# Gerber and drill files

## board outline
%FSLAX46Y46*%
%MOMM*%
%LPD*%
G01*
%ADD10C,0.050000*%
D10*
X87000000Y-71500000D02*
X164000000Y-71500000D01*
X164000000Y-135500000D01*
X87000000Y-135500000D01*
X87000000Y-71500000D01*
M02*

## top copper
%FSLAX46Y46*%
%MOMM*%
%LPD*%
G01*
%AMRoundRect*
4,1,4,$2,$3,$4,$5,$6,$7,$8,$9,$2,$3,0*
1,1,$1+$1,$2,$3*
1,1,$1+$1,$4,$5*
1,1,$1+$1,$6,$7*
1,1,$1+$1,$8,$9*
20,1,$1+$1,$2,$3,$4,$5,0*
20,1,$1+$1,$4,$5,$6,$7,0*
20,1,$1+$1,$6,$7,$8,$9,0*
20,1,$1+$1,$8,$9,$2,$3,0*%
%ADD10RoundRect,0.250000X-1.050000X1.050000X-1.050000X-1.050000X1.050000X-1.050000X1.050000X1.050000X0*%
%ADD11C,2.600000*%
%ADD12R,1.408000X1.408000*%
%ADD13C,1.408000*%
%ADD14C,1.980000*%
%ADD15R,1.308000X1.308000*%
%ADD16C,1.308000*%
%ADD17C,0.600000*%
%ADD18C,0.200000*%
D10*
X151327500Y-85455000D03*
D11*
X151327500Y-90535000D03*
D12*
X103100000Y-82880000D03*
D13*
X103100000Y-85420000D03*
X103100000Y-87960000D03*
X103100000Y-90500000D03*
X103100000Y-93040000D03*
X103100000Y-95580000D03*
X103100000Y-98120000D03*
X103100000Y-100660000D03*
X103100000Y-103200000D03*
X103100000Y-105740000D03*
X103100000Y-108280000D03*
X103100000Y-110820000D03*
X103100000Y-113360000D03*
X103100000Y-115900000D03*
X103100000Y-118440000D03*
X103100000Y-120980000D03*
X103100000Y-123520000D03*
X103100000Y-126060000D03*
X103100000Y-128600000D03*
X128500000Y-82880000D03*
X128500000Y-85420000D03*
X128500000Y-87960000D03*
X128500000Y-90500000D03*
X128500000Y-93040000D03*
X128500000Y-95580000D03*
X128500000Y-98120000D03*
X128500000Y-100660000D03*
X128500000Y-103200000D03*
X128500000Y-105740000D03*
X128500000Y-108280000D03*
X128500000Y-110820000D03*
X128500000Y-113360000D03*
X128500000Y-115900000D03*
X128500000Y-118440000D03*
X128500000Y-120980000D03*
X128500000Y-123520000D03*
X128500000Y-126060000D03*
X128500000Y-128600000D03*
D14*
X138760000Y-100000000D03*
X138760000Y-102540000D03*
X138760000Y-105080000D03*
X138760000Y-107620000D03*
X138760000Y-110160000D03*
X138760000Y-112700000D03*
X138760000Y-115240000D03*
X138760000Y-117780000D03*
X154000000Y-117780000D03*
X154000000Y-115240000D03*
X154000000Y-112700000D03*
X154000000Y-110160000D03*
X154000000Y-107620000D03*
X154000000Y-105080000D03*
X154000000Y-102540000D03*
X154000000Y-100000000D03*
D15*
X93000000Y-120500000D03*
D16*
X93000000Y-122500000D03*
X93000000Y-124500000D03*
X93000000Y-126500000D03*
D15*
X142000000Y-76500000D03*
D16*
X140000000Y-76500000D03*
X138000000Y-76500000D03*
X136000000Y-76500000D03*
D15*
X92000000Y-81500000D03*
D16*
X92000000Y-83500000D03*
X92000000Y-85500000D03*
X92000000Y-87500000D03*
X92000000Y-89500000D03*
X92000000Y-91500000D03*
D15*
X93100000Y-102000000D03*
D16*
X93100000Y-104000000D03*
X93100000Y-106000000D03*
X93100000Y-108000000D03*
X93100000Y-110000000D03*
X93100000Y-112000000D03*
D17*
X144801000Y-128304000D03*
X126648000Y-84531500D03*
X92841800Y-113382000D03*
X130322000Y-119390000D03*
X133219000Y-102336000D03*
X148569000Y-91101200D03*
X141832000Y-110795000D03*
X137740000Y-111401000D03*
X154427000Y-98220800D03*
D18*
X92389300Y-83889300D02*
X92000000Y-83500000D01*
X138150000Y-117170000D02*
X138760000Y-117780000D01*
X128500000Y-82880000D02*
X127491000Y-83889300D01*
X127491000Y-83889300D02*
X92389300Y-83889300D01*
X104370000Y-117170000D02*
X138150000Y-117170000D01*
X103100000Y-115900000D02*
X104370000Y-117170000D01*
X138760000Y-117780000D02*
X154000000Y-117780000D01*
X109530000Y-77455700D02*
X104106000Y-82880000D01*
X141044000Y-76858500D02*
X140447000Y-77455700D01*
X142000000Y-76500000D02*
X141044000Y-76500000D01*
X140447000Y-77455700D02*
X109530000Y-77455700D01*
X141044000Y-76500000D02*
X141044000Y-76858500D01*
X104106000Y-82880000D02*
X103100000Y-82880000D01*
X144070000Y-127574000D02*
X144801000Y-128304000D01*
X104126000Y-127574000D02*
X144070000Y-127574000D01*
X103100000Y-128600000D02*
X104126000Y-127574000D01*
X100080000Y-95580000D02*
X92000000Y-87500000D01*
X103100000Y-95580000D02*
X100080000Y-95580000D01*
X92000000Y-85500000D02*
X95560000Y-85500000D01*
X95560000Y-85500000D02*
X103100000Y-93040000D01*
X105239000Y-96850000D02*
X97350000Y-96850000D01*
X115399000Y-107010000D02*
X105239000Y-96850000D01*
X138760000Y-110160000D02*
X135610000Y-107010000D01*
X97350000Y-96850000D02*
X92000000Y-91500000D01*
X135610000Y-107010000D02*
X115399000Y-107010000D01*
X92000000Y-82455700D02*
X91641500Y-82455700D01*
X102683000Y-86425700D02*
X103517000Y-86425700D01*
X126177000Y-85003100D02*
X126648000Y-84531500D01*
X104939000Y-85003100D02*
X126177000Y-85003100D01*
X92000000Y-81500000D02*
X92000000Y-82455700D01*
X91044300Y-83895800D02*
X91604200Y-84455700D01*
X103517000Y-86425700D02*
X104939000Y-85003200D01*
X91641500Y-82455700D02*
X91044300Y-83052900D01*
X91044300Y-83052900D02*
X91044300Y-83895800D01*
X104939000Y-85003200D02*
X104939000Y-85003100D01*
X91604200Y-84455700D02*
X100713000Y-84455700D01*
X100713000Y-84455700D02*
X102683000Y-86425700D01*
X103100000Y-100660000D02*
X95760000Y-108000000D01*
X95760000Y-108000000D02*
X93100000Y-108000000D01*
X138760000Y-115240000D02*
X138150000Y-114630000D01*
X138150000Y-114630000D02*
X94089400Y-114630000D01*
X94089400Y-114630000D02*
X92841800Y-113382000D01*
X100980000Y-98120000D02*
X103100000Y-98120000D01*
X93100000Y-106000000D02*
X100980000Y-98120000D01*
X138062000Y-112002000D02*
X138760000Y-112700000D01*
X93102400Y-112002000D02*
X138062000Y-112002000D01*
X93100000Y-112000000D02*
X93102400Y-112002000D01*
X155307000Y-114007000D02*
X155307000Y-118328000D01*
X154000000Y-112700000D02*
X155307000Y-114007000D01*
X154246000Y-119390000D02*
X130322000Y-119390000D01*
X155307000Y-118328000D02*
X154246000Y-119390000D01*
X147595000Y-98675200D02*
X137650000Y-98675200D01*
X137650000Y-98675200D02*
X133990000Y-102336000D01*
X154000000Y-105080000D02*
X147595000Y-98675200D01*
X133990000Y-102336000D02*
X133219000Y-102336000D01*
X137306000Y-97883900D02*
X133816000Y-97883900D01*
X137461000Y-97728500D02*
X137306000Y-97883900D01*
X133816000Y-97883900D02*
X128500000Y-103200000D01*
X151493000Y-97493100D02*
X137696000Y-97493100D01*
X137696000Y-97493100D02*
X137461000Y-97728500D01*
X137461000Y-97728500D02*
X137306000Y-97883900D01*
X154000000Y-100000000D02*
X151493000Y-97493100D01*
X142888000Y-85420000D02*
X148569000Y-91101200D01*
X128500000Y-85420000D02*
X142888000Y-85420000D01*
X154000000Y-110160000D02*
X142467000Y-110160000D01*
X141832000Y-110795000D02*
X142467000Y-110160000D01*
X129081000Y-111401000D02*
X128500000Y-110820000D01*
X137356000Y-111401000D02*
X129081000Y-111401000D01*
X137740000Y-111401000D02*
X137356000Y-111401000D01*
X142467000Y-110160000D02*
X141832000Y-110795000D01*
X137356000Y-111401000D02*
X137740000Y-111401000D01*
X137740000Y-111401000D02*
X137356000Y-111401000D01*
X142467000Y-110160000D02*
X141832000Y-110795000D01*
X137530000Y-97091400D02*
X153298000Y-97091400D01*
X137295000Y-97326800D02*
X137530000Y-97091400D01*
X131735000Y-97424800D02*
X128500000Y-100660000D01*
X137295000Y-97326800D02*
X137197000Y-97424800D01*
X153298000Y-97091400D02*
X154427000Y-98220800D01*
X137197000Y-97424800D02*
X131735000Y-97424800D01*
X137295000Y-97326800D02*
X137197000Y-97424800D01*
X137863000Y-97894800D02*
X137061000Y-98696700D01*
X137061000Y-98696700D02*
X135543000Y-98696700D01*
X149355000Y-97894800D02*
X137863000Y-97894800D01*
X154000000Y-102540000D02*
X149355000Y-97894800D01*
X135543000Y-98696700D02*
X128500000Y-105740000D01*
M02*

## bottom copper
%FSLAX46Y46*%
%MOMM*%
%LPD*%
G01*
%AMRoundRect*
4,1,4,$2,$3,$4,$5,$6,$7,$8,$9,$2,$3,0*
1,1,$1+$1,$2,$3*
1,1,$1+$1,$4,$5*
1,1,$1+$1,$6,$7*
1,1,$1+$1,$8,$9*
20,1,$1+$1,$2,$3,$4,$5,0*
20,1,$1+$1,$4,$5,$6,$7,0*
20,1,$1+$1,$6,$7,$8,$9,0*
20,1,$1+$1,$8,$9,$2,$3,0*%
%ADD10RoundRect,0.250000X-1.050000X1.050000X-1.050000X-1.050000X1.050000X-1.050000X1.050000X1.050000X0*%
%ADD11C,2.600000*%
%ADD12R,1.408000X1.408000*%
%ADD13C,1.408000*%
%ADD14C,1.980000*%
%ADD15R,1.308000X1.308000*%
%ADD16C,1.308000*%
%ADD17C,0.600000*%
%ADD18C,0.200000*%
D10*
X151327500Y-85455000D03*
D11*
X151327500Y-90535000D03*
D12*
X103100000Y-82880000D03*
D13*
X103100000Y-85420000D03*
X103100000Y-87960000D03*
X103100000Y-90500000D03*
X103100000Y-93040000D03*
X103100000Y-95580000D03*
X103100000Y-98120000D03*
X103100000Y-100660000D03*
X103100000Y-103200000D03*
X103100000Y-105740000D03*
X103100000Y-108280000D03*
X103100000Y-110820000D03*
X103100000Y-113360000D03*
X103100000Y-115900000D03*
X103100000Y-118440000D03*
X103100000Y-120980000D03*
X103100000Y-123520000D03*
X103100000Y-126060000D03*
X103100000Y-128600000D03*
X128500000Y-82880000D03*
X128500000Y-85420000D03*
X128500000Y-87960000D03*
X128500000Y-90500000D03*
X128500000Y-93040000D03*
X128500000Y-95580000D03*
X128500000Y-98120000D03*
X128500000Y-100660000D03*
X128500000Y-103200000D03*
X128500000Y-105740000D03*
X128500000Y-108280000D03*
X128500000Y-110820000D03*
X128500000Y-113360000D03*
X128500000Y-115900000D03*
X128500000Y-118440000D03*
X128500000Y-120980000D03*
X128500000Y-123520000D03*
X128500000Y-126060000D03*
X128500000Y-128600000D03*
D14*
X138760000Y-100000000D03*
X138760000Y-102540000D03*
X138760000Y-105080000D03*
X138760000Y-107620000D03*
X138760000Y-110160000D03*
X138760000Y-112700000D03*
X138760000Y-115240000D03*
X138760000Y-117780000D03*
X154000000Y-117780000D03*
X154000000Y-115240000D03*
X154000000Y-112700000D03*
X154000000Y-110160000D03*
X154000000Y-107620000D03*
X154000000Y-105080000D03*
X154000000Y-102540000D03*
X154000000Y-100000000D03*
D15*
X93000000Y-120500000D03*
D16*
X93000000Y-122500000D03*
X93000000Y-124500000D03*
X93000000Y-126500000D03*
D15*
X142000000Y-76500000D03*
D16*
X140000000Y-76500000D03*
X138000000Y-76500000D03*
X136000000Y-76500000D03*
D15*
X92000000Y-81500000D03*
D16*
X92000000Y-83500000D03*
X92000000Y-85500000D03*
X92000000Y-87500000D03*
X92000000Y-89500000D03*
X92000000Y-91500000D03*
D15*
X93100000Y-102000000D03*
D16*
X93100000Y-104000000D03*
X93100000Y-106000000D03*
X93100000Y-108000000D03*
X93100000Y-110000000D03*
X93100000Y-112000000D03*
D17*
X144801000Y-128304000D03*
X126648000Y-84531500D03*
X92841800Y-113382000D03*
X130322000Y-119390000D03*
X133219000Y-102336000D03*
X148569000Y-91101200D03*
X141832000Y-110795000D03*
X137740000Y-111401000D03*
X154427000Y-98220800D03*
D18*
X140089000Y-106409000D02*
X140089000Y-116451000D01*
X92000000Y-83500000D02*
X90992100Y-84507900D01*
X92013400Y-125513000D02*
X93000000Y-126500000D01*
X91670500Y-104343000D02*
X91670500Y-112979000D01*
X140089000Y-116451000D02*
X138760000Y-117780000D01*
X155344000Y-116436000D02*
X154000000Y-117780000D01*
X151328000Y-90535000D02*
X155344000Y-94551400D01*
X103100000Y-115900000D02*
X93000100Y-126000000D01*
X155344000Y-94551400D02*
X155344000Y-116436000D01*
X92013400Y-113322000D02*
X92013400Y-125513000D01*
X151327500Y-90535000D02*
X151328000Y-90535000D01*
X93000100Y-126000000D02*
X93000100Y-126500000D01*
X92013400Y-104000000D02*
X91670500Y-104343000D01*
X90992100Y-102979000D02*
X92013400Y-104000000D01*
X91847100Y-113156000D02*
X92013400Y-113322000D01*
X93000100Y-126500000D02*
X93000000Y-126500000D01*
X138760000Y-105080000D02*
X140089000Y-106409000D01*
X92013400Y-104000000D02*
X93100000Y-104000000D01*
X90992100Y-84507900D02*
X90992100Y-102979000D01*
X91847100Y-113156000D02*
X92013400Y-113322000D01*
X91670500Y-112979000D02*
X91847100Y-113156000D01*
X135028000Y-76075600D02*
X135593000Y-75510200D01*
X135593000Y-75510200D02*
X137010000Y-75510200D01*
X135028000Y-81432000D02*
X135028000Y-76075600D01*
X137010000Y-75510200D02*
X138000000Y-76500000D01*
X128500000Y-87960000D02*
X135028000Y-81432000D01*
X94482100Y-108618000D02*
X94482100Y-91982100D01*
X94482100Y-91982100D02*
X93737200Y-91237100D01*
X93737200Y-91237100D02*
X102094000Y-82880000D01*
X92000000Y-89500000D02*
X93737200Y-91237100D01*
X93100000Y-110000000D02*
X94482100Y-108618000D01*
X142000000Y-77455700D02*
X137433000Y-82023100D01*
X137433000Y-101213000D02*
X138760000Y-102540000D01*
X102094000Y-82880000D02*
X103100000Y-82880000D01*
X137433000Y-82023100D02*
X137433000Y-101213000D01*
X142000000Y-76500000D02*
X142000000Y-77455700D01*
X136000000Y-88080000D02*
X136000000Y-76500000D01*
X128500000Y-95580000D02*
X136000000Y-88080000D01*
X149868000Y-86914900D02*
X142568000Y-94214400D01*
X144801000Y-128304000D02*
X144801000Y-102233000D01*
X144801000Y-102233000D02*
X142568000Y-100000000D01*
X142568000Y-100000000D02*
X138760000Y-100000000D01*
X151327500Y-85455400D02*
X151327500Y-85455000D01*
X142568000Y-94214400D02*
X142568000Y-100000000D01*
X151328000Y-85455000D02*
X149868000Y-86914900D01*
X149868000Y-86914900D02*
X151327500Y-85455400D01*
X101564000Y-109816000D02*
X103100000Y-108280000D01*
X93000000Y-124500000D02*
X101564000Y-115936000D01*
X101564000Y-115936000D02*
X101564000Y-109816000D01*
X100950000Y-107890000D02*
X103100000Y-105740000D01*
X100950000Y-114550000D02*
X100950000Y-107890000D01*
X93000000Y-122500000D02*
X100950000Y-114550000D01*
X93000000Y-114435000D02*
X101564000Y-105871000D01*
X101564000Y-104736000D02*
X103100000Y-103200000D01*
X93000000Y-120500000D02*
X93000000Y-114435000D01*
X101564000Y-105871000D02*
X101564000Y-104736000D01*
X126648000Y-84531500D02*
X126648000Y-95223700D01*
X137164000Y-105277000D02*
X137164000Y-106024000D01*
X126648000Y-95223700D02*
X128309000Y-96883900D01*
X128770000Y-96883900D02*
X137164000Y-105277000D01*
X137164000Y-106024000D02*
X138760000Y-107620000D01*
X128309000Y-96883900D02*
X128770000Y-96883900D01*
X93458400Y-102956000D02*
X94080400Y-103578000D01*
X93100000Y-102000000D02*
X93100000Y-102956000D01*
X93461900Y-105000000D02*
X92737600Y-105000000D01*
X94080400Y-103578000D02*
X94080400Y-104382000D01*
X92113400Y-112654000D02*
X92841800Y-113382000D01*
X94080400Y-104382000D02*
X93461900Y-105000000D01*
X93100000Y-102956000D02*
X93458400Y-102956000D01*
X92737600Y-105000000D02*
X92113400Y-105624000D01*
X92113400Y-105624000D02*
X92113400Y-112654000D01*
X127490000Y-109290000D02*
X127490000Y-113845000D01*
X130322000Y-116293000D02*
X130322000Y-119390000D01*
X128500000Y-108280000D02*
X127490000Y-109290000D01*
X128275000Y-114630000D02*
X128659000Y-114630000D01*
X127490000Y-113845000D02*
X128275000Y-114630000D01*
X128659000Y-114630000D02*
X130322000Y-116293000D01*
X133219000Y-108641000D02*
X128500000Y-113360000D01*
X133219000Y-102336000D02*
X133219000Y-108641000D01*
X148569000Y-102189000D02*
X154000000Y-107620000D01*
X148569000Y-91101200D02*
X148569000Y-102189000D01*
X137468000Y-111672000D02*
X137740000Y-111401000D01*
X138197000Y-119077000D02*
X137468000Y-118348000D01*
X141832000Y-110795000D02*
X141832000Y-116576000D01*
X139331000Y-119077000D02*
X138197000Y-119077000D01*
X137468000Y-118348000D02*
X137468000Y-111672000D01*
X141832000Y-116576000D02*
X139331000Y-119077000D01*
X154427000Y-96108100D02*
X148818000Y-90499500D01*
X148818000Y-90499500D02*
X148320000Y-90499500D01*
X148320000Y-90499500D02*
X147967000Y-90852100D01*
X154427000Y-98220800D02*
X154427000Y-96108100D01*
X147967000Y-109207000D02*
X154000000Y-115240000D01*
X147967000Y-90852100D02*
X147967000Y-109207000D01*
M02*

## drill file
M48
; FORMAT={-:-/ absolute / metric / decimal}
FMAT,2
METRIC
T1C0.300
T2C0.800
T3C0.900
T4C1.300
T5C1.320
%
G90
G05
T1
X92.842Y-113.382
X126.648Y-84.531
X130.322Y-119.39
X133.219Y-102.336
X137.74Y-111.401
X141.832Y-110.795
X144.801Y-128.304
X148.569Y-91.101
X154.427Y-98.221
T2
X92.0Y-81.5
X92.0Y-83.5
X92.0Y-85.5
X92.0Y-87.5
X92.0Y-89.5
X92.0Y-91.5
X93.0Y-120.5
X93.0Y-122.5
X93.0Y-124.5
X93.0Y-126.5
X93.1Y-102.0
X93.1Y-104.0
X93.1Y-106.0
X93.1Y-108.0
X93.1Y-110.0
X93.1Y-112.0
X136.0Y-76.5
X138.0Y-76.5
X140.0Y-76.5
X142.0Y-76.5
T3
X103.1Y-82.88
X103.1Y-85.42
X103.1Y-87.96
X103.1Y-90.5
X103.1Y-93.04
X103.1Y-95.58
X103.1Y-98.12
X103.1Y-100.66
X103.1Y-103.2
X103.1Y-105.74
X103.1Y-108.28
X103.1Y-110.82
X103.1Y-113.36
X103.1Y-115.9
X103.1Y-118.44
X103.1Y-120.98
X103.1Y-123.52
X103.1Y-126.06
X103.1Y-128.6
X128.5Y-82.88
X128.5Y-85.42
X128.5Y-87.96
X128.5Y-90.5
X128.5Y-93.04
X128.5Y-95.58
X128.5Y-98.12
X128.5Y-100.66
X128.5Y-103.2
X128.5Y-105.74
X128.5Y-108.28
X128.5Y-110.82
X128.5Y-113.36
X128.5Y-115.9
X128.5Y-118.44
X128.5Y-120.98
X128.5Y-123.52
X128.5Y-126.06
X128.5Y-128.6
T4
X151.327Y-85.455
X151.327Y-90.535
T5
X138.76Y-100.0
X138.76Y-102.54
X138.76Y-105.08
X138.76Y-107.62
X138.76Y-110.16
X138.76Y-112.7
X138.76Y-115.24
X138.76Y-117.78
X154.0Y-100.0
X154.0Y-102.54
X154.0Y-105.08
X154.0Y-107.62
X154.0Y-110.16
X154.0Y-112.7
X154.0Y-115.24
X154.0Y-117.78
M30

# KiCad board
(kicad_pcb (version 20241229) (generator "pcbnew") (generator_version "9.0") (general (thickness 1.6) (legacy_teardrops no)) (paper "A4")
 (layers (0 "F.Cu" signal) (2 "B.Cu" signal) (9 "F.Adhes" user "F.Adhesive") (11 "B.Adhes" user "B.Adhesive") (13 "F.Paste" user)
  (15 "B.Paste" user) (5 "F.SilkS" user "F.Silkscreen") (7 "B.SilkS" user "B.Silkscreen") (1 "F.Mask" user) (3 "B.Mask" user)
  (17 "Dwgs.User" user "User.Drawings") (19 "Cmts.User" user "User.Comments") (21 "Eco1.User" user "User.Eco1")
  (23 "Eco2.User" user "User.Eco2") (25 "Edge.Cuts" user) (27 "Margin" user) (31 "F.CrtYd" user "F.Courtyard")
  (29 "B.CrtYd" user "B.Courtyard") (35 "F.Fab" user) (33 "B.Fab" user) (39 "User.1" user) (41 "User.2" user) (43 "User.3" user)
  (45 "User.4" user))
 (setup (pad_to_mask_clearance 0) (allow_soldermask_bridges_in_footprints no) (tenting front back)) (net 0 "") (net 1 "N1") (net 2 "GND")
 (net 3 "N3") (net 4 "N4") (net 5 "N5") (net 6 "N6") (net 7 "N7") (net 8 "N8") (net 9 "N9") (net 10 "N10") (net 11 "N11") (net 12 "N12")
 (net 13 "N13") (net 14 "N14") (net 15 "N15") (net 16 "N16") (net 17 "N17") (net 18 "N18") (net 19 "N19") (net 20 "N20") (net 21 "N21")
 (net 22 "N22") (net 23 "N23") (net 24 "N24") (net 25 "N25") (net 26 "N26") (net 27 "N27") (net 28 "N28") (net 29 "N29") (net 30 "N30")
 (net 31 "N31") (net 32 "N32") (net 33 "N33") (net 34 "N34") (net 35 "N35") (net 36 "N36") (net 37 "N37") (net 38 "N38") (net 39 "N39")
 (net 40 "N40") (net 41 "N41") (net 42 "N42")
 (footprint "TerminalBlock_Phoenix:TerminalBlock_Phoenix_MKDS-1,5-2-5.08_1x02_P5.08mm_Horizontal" (layer "F.Cu") (at 151.3275 85.455 -90)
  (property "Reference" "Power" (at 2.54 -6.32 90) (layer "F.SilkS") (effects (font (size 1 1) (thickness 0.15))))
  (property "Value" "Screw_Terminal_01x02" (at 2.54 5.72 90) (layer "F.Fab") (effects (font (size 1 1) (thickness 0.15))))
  (pad "1" thru_hole roundrect (at 0 0 270) (size 2.6 2.6) (drill 1.3) (layers "*.Cu" "*.Mask") (remove_unused_layers no)
   (roundrect_rratio 0.096154) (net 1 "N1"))
  (pad "2" thru_hole circle (at 5.08 0 270) (size 2.6 2.6) (drill 1.3) (layers "*.Cu" "*.Mask") (remove_unused_layers no) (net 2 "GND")))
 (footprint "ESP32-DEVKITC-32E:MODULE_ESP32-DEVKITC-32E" (layer "F.Cu") (at 115.8 105.715)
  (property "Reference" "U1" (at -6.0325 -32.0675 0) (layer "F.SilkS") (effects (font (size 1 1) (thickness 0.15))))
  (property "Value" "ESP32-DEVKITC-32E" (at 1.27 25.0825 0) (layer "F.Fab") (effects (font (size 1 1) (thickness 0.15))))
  (pad "J2_1" thru_hole rect (at -12.7 -22.835) (size 1.408 1.408) (drill 0.9) (layers "*.Cu" "*.Mask") (remove_unused_layers no)
   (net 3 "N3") (solder_mask_margin 0.102))
  (pad "J2_2" thru_hole circle (at -12.7 -20.295) (size 1.408 1.408) (drill 0.9) (layers "*.Cu" "*.Mask") (remove_unused_layers no)
   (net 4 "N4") (solder_mask_margin 0.102))
  (pad "J2_3" thru_hole circle (at -12.7 -17.755) (size 1.408 1.408) (drill 0.9) (layers "*.Cu" "*.Mask") (remove_unused_layers no)
   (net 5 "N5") (solder_mask_margin 0.102))
  (pad "J2_4" thru_hole circle (at -12.7 -15.215) (size 1.408 1.408) (drill 0.9) (layers "*.Cu" "*.Mask") (remove_unused_layers no)
   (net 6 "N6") (solder_mask_margin 0.102))
  (pad "J2_5" thru_hole circle (at -12.7 -12.675) (size 1.408 1.408) (drill 0.9) (layers "*.Cu" "*.Mask") (remove_unused_layers no)
   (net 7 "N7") (solder_mask_margin 0.102))
  (pad "J2_6" thru_hole circle (at -12.7 -10.135) (size 1.408 1.408) (drill 0.9) (layers "*.Cu" "*.Mask") (remove_unused_layers no)
   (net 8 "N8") (solder_mask_margin 0.102))
  (pad "J2_7" thru_hole circle (at -12.7 -7.595) (size 1.408 1.408) (drill 0.9) (layers "*.Cu" "*.Mask") (remove_unused_layers no)
   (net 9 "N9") (solder_mask_margin 0.102))
  (pad "J2_8" thru_hole circle (at -12.7 -5.055) (size 1.408 1.408) (drill 0.9) (layers "*.Cu" "*.Mask") (remove_unused_layers no)
   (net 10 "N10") (solder_mask_margin 0.102))
  (pad "J2_9" thru_hole circle (at -12.7 -2.515) (size 1.408 1.408) (drill 0.9) (layers "*.Cu" "*.Mask") (remove_unused_layers no)
   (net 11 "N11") (solder_mask_margin 0.102))
  (pad "J2_10" thru_hole circle (at -12.7 0.025) (size 1.408 1.408) (drill 0.9) (layers "*.Cu" "*.Mask") (remove_unused_layers no)
   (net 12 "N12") (solder_mask_margin 0.102))
  (pad "J2_11" thru_hole circle (at -12.7 2.565) (size 1.408 1.408) (drill 0.9) (layers "*.Cu" "*.Mask") (remove_unused_layers no)
   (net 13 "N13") (solder_mask_margin 0.102))
  (pad "J2_12" thru_hole circle (at -12.7 5.105) (size 1.408 1.408) (drill 0.9) (layers "*.Cu" "*.Mask") (remove_unused_layers no)
   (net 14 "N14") (solder_mask_margin 0.102))
  (pad "J2_13" thru_hole circle (at -12.7 7.645) (size 1.408 1.408) (drill 0.9) (layers "*.Cu" "*.Mask") (remove_unused_layers no)
   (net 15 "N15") (solder_mask_margin 0.102))
  (pad "J2_14" thru_hole circle (at -12.7 10.185) (size 1.408 1.408) (drill 0.9) (layers "*.Cu" "*.Mask") (remove_unused_layers no)
   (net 2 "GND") (solder_mask_margin 0.102))
  (pad "J2_15" thru_hole circle (at -12.7 12.725) (size 1.408 1.408) (drill 0.9) (layers "*.Cu" "*.Mask") (remove_unused_layers no)
   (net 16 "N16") (solder_mask_margin 0.102))
  (pad "J2_16" thru_hole circle (at -12.7 15.265) (size 1.408 1.408) (drill 0.9) (layers "*.Cu" "*.Mask") (remove_unused_layers no)
   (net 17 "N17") (solder_mask_margin 0.102))
  (pad "J2_17" thru_hole circle (at -12.7 17.805) (size 1.408 1.408) (drill 0.9) (layers "*.Cu" "*.Mask") (remove_unused_layers no)
   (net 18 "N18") (solder_mask_margin 0.102))
  (pad "J2_18" thru_hole circle (at -12.7 20.345) (size 1.408 1.408) (drill 0.9) (layers "*.Cu" "*.Mask") (remove_unused_layers no)
   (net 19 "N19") (solder_mask_margin 0.102))
  (pad "J2_19" thru_hole circle (at -12.7 22.885) (size 1.408 1.408) (drill 0.9) (layers "*.Cu" "*.Mask") (remove_unused_layers no)
   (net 1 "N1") (solder_mask_margin 0.102))
  (pad "J3_1" thru_hole circle (at 12.7 -22.835) (size 1.408 1.408) (drill 0.9) (layers "*.Cu" "*.Mask") (remove_unused_layers no)
   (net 2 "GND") (solder_mask_margin 0.102))
  (pad "J3_2" thru_hole circle (at 12.7 -20.295) (size 1.408 1.408) (drill 0.9) (layers "*.Cu" "*.Mask") (remove_unused_layers no)
   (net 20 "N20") (solder_mask_margin 0.102))
  (pad "J3_3" thru_hole circle (at 12.7 -17.755) (size 1.408 1.408) (drill 0.9) (layers "*.Cu" "*.Mask") (remove_unused_layers no)
   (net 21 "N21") (solder_mask_margin 0.102))
  (pad "J3_4" thru_hole circle (at 12.7 -15.215) (size 1.408 1.408) (drill 0.9) (layers "*.Cu" "*.Mask") (remove_unused_layers no)
   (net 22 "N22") (solder_mask_margin 0.102))
  (pad "J3_5" thru_hole circle (at 12.7 -12.675) (size 1.408 1.408) (drill 0.9) (layers "*.Cu" "*.Mask") (remove_unused_layers no)
   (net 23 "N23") (solder_mask_margin 0.102))
  (pad "J3_6" thru_hole circle (at 12.7 -10.135) (size 1.408 1.408) (drill 0.9) (layers "*.Cu" "*.Mask") (remove_unused_layers no)
   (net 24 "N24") (solder_mask_margin 0.102))
  (pad "J3_7" thru_hole circle (at 12.7 -7.595) (size 1.408 1.408) (drill 0.9) (layers "*.Cu" "*.Mask") (remove_unused_layers no)
   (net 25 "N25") (solder_mask_margin 0.102))
  (pad "J3_8" thru_hole circle (at 12.7 -5.055) (size 1.408 1.408) (drill 0.9) (layers "*.Cu" "*.Mask") (remove_unused_layers no)
   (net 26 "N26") (solder_mask_margin 0.102))
  (pad "J3_9" thru_hole circle (at 12.7 -2.515) (size 1.408 1.408) (drill 0.9) (layers "*.Cu" "*.Mask") (remove_unused_layers no)
   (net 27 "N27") (solder_mask_margin 0.102))
  (pad "J3_10" thru_hole circle (at 12.7 0.025) (size 1.408 1.408) (drill 0.9) (layers "*.Cu" "*.Mask") (remove_unused_layers no)
   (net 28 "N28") (solder_mask_margin 0.102))
  (pad "J3_11" thru_hole circle (at 12.7 2.565) (size 1.408 1.408) (drill 0.9) (layers "*.Cu" "*.Mask") (remove_unused_layers no)
   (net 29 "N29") (solder_mask_margin 0.102))
  (pad "J3_12" thru_hole circle (at 12.7 5.105) (size 1.408 1.408) (drill 0.9) (layers "*.Cu" "*.Mask") (remove_unused_layers no)
   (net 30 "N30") (solder_mask_margin 0.102))
  (pad "J3_13" thru_hole circle (at 12.7 7.645) (size 1.408 1.408) (drill 0.9) (layers "*.Cu" "*.Mask") (remove_unused_layers no)
   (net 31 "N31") (solder_mask_margin 0.102))
  (pad "J3_14" thru_hole circle (at 12.7 10.185) (size 1.408 1.408) (drill 0.9) (layers "*.Cu" "*.Mask") (remove_unused_layers no)
   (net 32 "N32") (solder_mask_margin 0.102))
  (pad "J3_15" thru_hole circle (at 12.7 12.725) (size 1.408 1.408) (drill 0.9) (layers "*.Cu" "*.Mask") (remove_unused_layers no)
   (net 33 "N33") (solder_mask_margin 0.102))
  (pad "J3_16" thru_hole circle (at 12.7 15.265) (size 1.408 1.408) (drill 0.9) (layers "*.Cu" "*.Mask") (remove_unused_layers no)
   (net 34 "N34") (solder_mask_margin 0.102))
  (pad "J3_17" thru_hole circle (at 12.7 17.805) (size 1.408 1.408) (drill 0.9) (layers "*.Cu" "*.Mask") (remove_unused_layers no)
   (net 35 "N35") (solder_mask_margin 0.102))
  (pad "J3_18" thru_hole circle (at 12.7 20.345) (size 1.408 1.408) (drill 0.9) (layers "*.Cu" "*.Mask") (remove_unused_layers no)
   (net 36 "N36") (solder_mask_margin 0.102))
  (pad "J3_19" thru_hole circle (at 12.7 22.885) (size 1.408 1.408) (drill 0.9) (layers "*.Cu" "*.Mask") (remove_unused_layers no)
   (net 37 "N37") (solder_mask_margin 0.102)))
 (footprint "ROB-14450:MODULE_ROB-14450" (layer "F.Cu") (at 146.38 108.89)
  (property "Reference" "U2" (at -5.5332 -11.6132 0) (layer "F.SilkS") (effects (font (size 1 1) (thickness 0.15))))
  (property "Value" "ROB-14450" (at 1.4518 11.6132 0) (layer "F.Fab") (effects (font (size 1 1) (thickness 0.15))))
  (pad "1" thru_hole circle (at -7.62 -8.89) (size 1.98 1.98) (drill 1.32) (layers "*.Cu" "*.Mask") (remove_unused_layers no) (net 1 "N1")
   (solder_mask_margin 0.102))
  (pad "2" thru_hole circle (at -7.62 -6.35) (size 1.98 1.98) (drill 1.32) (layers "*.Cu" "*.Mask") (remove_unused_layers no) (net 3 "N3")
   (solder_mask_margin 0.102))
  (pad "3" thru_hole circle (at -7.62 -3.81) (size 1.98 1.98) (drill 1.32) (layers "*.Cu" "*.Mask") (remove_unused_layers no) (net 2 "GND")
   (solder_mask_margin 0.102))
  (pad "4" thru_hole circle (at -7.62 -1.27) (size 1.98 1.98) (drill 1.32) (layers "*.Cu" "*.Mask") (remove_unused_layers no) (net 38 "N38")
   (solder_mask_margin 0.102))
  (pad "5" thru_hole circle (at -7.62 1.27) (size 1.98 1.98) (drill 1.32) (layers "*.Cu" "*.Mask") (remove_unused_layers no) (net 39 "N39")
   (solder_mask_margin 0.102))
  (pad "6" thru_hole circle (at -7.62 3.81) (size 1.98 1.98) (drill 1.32) (layers "*.Cu" "*.Mask") (remove_unused_layers no) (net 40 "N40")
   (solder_mask_margin 0.102))
  (pad "7" thru_hole circle (at -7.62 6.35) (size 1.98 1.98) (drill 1.32) (layers "*.Cu" "*.Mask") (remove_unused_layers no) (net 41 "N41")
   (solder_mask_margin 0.102))
  (pad "8" thru_hole circle (at -7.62 8.89) (size 1.98 1.98) (drill 1.32) (layers "*.Cu" "*.Mask") (remove_unused_layers no) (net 2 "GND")
   (solder_mask_margin 0.102))
  (pad "9" thru_hole circle (at 7.62 8.89) (size 1.98 1.98) (drill 1.32) (layers "*.Cu" "*.Mask") (remove_unused_layers no) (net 2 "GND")
   (solder_mask_margin 0.102))
  (pad "10" thru_hole circle (at 7.62 6.35) (size 1.98 1.98) (drill 1.32) (layers "*.Cu" "*.Mask") (remove_unused_layers no) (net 26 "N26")
   (solder_mask_margin 0.102))
  (pad "11" thru_hole circle (at 7.62 3.81) (size 1.98 1.98) (drill 1.32) (layers "*.Cu" "*.Mask") (remove_unused_layers no) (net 29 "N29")
   (solder_mask_margin 0.102))
  (pad "12" thru_hole circle (at 7.62 1.27) (size 1.98 1.98) (drill 1.32) (layers "*.Cu" "*.Mask") (remove_unused_layers no) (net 30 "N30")
   (solder_mask_margin 0.102))
  (pad "13" thru_hole circle (at 7.62 -1.27) (size 1.98 1.98) (drill 1.32) (layers "*.Cu" "*.Mask") (remove_unused_layers no) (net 20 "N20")
   (solder_mask_margin 0.102))
  (pad "14" thru_hole circle (at 7.62 -3.81) (size 1.98 1.98) (drill 1.32) (layers "*.Cu" "*.Mask") (remove_unused_layers no) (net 31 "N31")
   (solder_mask_margin 0.102))
  (pad "15" thru_hole circle (at 7.62 -6.35) (size 1.98 1.98) (drill 1.32) (layers "*.Cu" "*.Mask") (remove_unused_layers no) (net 28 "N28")
   (solder_mask_margin 0.102))
  (pad "16" thru_hole circle (at 7.62 -8.89) (size 1.98 1.98) (drill 1.32) (layers "*.Cu" "*.Mask") (remove_unused_layers no) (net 27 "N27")
   (solder_mask_margin 0.102)))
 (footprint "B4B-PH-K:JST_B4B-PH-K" (layer "F.Cu") (at 92.45 123.5 90)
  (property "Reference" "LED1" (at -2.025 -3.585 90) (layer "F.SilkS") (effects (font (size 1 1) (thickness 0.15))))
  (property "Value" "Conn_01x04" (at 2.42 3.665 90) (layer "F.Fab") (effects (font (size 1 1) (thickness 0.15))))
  (pad "1" thru_hole rect (at 3 0.55 90) (size 1.308 1.308) (drill 0.8) (layers "*.Cu" "*.Mask") (remove_unused_layers no) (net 11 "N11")
   (solder_mask_margin 0.102))
  (pad "2" thru_hole circle (at 1 0.55 90) (size 1.308 1.308) (drill 0.8) (layers "*.Cu" "*.Mask") (remove_unused_layers no) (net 12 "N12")
   (solder_mask_margin 0.102))
  (pad "3" thru_hole circle (at -1 0.55 90) (size 1.308 1.308) (drill 0.8) (layers "*.Cu" "*.Mask") (remove_unused_layers no) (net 13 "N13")
   (solder_mask_margin 0.102))
  (pad "4" thru_hole circle (at -3 0.55 90) (size 1.308 1.308) (drill 0.8) (layers "*.Cu" "*.Mask") (remove_unused_layers no) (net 2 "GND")
   (solder_mask_margin 0.102)))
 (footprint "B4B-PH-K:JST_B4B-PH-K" (layer "F.Cu") (at 139 75.95)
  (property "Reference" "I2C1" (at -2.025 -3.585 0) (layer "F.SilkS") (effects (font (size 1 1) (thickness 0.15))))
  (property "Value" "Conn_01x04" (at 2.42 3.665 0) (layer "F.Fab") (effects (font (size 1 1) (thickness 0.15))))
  (pad "1" thru_hole rect (at 3 0.55) (size 1.308 1.308) (drill 0.8) (layers "*.Cu" "*.Mask") (remove_unused_layers no) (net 3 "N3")
   (solder_mask_margin 0.102))
  (pad "2" thru_hole circle (at 1 0.55) (size 1.308 1.308) (drill 0.8) (layers "*.Cu" "*.Mask") (remove_unused_layers no) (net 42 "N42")
   (solder_mask_margin 0.102))
  (pad "3" thru_hole circle (at -1 0.55) (size 1.308 1.308) (drill 0.8) (layers "*.Cu" "*.Mask") (remove_unused_layers no) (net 21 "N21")
   (solder_mask_margin 0.102))
  (pad "4" thru_hole circle (at -3 0.55) (size 1.308 1.308) (drill 0.8) (layers "*.Cu" "*.Mask") (remove_unused_layers no) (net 24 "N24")
   (solder_mask_margin 0.102)))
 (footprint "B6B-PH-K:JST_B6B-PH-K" (layer "F.Cu") (at 91.45 86.5 90)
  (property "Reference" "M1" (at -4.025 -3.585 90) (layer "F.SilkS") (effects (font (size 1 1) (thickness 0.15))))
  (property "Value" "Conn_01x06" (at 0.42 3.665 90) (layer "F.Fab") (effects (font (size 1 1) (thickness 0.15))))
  (pad "1" thru_hole rect (at 5 0.55 90) (size 1.308 1.308) (drill 0.8) (layers "*.Cu" "*.Mask") (remove_unused_layers no) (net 38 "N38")
   (solder_mask_margin 0.102))
  (pad "2" thru_hole circle (at 3 0.55 90) (size 1.308 1.308) (drill 0.8) (layers "*.Cu" "*.Mask") (remove_unused_layers no) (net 2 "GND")
   (solder_mask_margin 0.102))
  (pad "3" thru_hole circle (at 1 0.55 90) (size 1.308 1.308) (drill 0.8) (layers "*.Cu" "*.Mask") (remove_unused_layers no) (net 7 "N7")
   (solder_mask_margin 0.102))
  (pad "4" thru_hole circle (at -1 0.55 90) (size 1.308 1.308) (drill 0.8) (layers "*.Cu" "*.Mask") (remove_unused_layers no) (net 8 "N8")
   (solder_mask_margin 0.102))
  (pad "5" thru_hole circle (at -3 0.55 90) (size 1.308 1.308) (drill 0.8) (layers "*.Cu" "*.Mask") (remove_unused_layers no) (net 3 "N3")
   (solder_mask_margin 0.102))
  (pad "6" thru_hole circle (at -5 0.55 90) (size 1.308 1.308) (drill 0.8) (layers "*.Cu" "*.Mask") (remove_unused_layers no) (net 39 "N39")
   (solder_mask_margin 0.102)))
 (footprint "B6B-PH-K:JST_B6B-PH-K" (layer "F.Cu") (at 92.55 107 90)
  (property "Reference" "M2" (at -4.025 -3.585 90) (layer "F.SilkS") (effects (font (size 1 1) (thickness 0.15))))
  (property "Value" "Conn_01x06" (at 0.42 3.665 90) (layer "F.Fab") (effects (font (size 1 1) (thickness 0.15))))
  (pad "1" thru_hole rect (at 5 0.55 90) (size 1.308 1.308) (drill 0.8) (layers "*.Cu" "*.Mask") (remove_unused_layers no) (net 41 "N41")
   (solder_mask_margin 0.102))
  (pad "2" thru_hole circle (at 3 0.55 90) (size 1.308 1.308) (drill 0.8) (layers "*.Cu" "*.Mask") (remove_unused_layers no) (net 2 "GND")
   (solder_mask_margin 0.102))
  (pad "3" thru_hole circle (at 1 0.55 90) (size 1.308 1.308) (drill 0.8) (layers "*.Cu" "*.Mask") (remove_unused_layers no) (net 9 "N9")
   (solder_mask_margin 0.102))
  (pad "4" thru_hole circle (at -1 0.55 90) (size 1.308 1.308) (drill 0.8) (layers "*.Cu" "*.Mask") (remove_unused_layers no) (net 10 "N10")
   (solder_mask_margin 0.102))
  (pad "5" thru_hole circle (at -3 0.55 90) (size 1.308 1.308) (drill 0.8) (layers "*.Cu" "*.Mask") (remove_unused_layers no) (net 3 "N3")
   (solder_mask_margin 0.102))
  (pad "6" thru_hole circle (at -5 0.55 90) (size 1.308 1.308) (drill 0.8) (layers "*.Cu" "*.Mask") (remove_unused_layers no) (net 40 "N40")
   (solder_mask_margin 0.102)))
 (gr_rect (start 87 71.5) (end 164 135.5) (stroke (width 0.05) (type solid)) (fill no) (layer "Edge.Cuts"))
 (segment (start 92.3893 83.8893) (end 92 83.5) (width 0.2) (layer "F.Cu") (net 2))
 (segment (start 138.15 117.17) (end 138.76 117.78) (width 0.2) (layer "F.Cu") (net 2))
 (segment (start 128.5 82.88) (end 127.491 83.8893) (width 0.2) (layer "F.Cu") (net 2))
 (segment (start 127.491 83.8893) (end 92.3893 83.8893) (width 0.2) (layer "F.Cu") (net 2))
 (segment (start 104.37 117.17) (end 138.15 117.17) (width 0.2) (layer "F.Cu") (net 2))
 (segment (start 103.1 115.9) (end 104.37 117.17) (width 0.2) (layer "F.Cu") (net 2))
 (segment (start 138.76 117.78) (end 154 117.78) (width 0.2) (layer "F.Cu") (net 2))
 (segment (start 140.089 106.409) (end 140.089 116.451) (width 0.2) (layer "B.Cu") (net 2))
 (segment (start 92 83.5) (end 90.9921 84.5079) (width 0.2) (layer "B.Cu") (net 2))
 (segment (start 92.0134 125.513) (end 93 126.5) (width 0.2) (layer "B.Cu") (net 2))
 (segment (start 91.6705 104.343) (end 91.6705 112.979) (width 0.2) (layer "B.Cu") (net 2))
 (segment (start 140.089 116.451) (end 138.76 117.78) (width 0.2) (layer "B.Cu") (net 2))
 (segment (start 155.344 116.436) (end 154 117.78) (width 0.2) (layer "B.Cu") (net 2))
 (segment (start 151.328 90.535) (end 155.344 94.5514) (width 0.2) (layer "B.Cu") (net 2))
 (segment (start 103.1 115.9) (end 93.0001 126) (width 0.2) (layer "B.Cu") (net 2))
 (segment (start 155.344 94.5514) (end 155.344 116.436) (width 0.2) (layer "B.Cu") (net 2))
 (segment (start 92.0134 113.322) (end 92.0134 125.513) (width 0.2) (layer "B.Cu") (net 2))
 (segment (start 151.3275 90.535) (end 151.328 90.535) (width 0.2) (layer "B.Cu") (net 2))
 (segment (start 93.0001 126) (end 93.0001 126.5) (width 0.2) (layer "B.Cu") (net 2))
 (segment (start 92.0134 104) (end 91.6705 104.343) (width 0.2) (layer "B.Cu") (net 2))
 (segment (start 90.9921 102.979) (end 92.0134 104) (width 0.2) (layer "B.Cu") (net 2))
 (segment (start 91.8471 113.156) (end 92.0134 113.322) (width 0.2) (layer "B.Cu") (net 2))
 (segment (start 93.0001 126.5) (end 93 126.5) (width 0.2) (layer "B.Cu") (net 2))
 (segment (start 138.76 105.08) (end 140.089 106.409) (width 0.2) (layer "B.Cu") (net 2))
 (segment (start 92.0134 104) (end 93.1 104) (width 0.2) (layer "B.Cu") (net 2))
 (segment (start 90.9921 84.5079) (end 90.9921 102.979) (width 0.2) (layer "B.Cu") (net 2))
 (segment (start 91.8471 113.156) (end 92.0134 113.322) (width 0.2) (layer "B.Cu") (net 2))
 (segment (start 91.6705 112.979) (end 91.8471 113.156) (width 0.2) (layer "B.Cu") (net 2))
 (segment (start 135.028 76.0756) (end 135.593 75.5102) (width 0.2) (layer "B.Cu") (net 21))
 (segment (start 135.593 75.5102) (end 137.01 75.5102) (width 0.2) (layer "B.Cu") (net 21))
 (segment (start 135.028 81.432) (end 135.028 76.0756) (width 0.2) (layer "B.Cu") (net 21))
 (segment (start 137.01 75.5102) (end 138 76.5) (width 0.2) (layer "B.Cu") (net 21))
 (segment (start 128.5 87.96) (end 135.028 81.432) (width 0.2) (layer "B.Cu") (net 21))
 (segment (start 109.53 77.4557) (end 104.106 82.88) (width 0.2) (layer "F.Cu") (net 3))
 (segment (start 141.044 76.8585) (end 140.447 77.4557) (width 0.2) (layer "F.Cu") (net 3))
 (segment (start 142 76.5) (end 141.044 76.5) (width 0.2) (layer "F.Cu") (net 3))
 (segment (start 140.447 77.4557) (end 109.53 77.4557) (width 0.2) (layer "F.Cu") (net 3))
 (segment (start 141.044 76.5) (end 141.044 76.8585) (width 0.2) (layer "F.Cu") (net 3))
 (segment (start 104.106 82.88) (end 103.1 82.88) (width 0.2) (layer "F.Cu") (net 3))
 (segment (start 94.4821 108.618) (end 94.4821 91.9821) (width 0.2) (layer "B.Cu") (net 3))
 (segment (start 94.4821 91.9821) (end 93.7372 91.2371) (width 0.2) (layer "B.Cu") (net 3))
 (segment (start 93.7372 91.2371) (end 102.094 82.88) (width 0.2) (layer "B.Cu") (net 3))
 (segment (start 92 89.5) (end 93.7372 91.2371) (width 0.2) (layer "B.Cu") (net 3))
 (segment (start 93.1 110) (end 94.4821 108.618) (width 0.2) (layer "B.Cu") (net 3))
 (segment (start 142 77.4557) (end 137.433 82.0231) (width 0.2) (layer "B.Cu") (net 3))
 (segment (start 137.433 101.213) (end 138.76 102.54) (width 0.2) (layer "B.Cu") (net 3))
 (segment (start 102.094 82.88) (end 103.1 82.88) (width 0.2) (layer "B.Cu") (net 3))
 (segment (start 137.433 82.0231) (end 137.433 101.213) (width 0.2) (layer "B.Cu") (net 3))
 (segment (start 142 76.5) (end 142 77.4557) (width 0.2) (layer "B.Cu") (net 3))
 (segment (start 136 88.08) (end 136 76.5) (width 0.2) (layer "B.Cu") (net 24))
 (segment (start 128.5 95.58) (end 136 88.08) (width 0.2) (layer "B.Cu") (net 24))
 (segment (start 144.07 127.574) (end 144.801 128.304) (width 0.2) (layer "F.Cu") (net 1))
 (segment (start 104.126 127.574) (end 144.07 127.574) (width 0.2) (layer "F.Cu") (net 1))
 (segment (start 103.1 128.6) (end 104.126 127.574) (width 0.2) (layer "F.Cu") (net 1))
 (via (at 144.801 128.304) (size 0.6) (drill 0.3) (layers "F.Cu" "B.Cu") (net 1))
 (segment (start 149.868 86.9149) (end 142.568 94.2144) (width 0.2) (layer "B.Cu") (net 1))
 (segment (start 144.801 128.304) (end 144.801 102.233) (width 0.2) (layer "B.Cu") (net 1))
 (segment (start 144.801 102.233) (end 142.568 100) (width 0.2) (layer "B.Cu") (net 1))
 (segment (start 142.568 100) (end 138.76 100) (width 0.2) (layer "B.Cu") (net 1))
 (segment (start 151.3275 85.4554) (end 151.3275 85.455) (width 0.2) (layer "B.Cu") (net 1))
 (segment (start 142.568 94.2144) (end 142.568 100) (width 0.2) (layer "B.Cu") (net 1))
 (segment (start 151.328 85.455) (end 149.868 86.9149) (width 0.2) (layer "B.Cu") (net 1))
 (segment (start 149.868 86.9149) (end 151.3275 85.4554) (width 0.2) (layer "B.Cu") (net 1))
 (segment (start 101.564 109.816) (end 103.1 108.28) (width 0.2) (layer "B.Cu") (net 13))
 (segment (start 93 124.5) (end 101.564 115.936) (width 0.2) (layer "B.Cu") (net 13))
 (segment (start 101.564 115.936) (end 101.564 109.816) (width 0.2) (layer "B.Cu") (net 13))
 (segment (start 100.95 107.89) (end 103.1 105.74) (width 0.2) (layer "B.Cu") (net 12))
 (segment (start 100.95 114.55) (end 100.95 107.89) (width 0.2) (layer "B.Cu") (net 12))
 (segment (start 93 122.5) (end 100.95 114.55) (width 0.2) (layer "B.Cu") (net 12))
 (segment (start 93 114.435) (end 101.564 105.871) (width 0.2) (layer "B.Cu") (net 11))
 (segment (start 101.564 104.736) (end 103.1 103.2) (width 0.2) (layer "B.Cu") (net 11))
 (segment (start 93 120.5) (end 93 114.435) (width 0.2) (layer "B.Cu") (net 11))
 (segment (start 101.564 105.871) (end 101.564 104.736) (width 0.2) (layer "B.Cu") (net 11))
 (segment (start 100.08 95.58) (end 92 87.5) (width 0.2) (layer "F.Cu") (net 8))
 (segment (start 103.1 95.58) (end 100.08 95.58) (width 0.2) (layer "F.Cu") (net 8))
 (segment (start 92 85.5) (end 95.56 85.5) (width 0.2) (layer "F.Cu") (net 7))
 (segment (start 95.56 85.5) (end 103.1 93.04) (width 0.2) (layer "F.Cu") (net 7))
 (segment (start 105.239 96.85) (end 97.35 96.85) (width 0.2) (layer "F.Cu") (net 39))
 (segment (start 115.399 107.01) (end 105.239 96.85) (width 0.2) (layer "F.Cu") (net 39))
 (segment (start 138.76 110.16) (end 135.61 107.01) (width 0.2) (layer "F.Cu") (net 39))
 (segment (start 97.35 96.85) (end 92 91.5) (width 0.2) (layer "F.Cu") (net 39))
 (segment (start 135.61 107.01) (end 115.399 107.01) (width 0.2) (layer "F.Cu") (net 39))
 (segment (start 92 82.4557) (end 91.6415 82.4557) (width 0.2) (layer "F.Cu") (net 38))
 (segment (start 102.683 86.4257) (end 103.517 86.4257) (width 0.2) (layer "F.Cu") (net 38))
 (segment (start 126.177 85.0031) (end 126.648 84.5315) (width 0.2) (layer "F.Cu") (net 38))
 (segment (start 104.939 85.0031) (end 126.177 85.0031) (width 0.2) (layer "F.Cu") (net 38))
 (segment (start 92 81.5) (end 92 82.4557) (width 0.2) (layer "F.Cu") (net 38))
 (segment (start 91.0443 83.8958) (end 91.6042 84.4557) (width 0.2) (layer "F.Cu") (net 38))
 (segment (start 103.517 86.4257) (end 104.939 85.0032) (width 0.2) (layer "F.Cu") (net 38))
 (segment (start 91.6415 82.4557) (end 91.0443 83.0529) (width 0.2) (layer "F.Cu") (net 38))
 (segment (start 91.0443 83.0529) (end 91.0443 83.8958) (width 0.2) (layer "F.Cu") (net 38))
 (segment (start 104.939 85.0032) (end 104.939 85.0031) (width 0.2) (layer "F.Cu") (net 38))
 (segment (start 91.6042 84.4557) (end 100.713 84.4557) (width 0.2) (layer "F.Cu") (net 38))
 (segment (start 100.713 84.4557) (end 102.683 86.4257) (width 0.2) (layer "F.Cu") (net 38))
 (via (at 126.648 84.5315) (size 0.6) (drill 0.3) (layers "F.Cu" "B.Cu") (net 38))
 (segment (start 126.648 84.5315) (end 126.648 95.2237) (width 0.2) (layer "B.Cu") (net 38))
 (segment (start 137.164 105.277) (end 137.164 106.024) (width 0.2) (layer "B.Cu") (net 38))
 (segment (start 126.648 95.2237) (end 128.309 96.8839) (width 0.2) (layer "B.Cu") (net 38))
 (segment (start 128.77 96.8839) (end 137.164 105.277) (width 0.2) (layer "B.Cu") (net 38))
 (segment (start 137.164 106.024) (end 138.76 107.62) (width 0.2) (layer "B.Cu") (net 38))
 (segment (start 128.309 96.8839) (end 128.77 96.8839) (width 0.2) (layer "B.Cu") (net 38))
 (segment (start 103.1 100.66) (end 95.76 108) (width 0.2) (layer "F.Cu") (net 10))
 (segment (start 95.76 108) (end 93.1 108) (width 0.2) (layer "F.Cu") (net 10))
 (segment (start 138.76 115.24) (end 138.15 114.63) (width 0.2) (layer "F.Cu") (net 41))
 (segment (start 138.15 114.63) (end 94.0894 114.63) (width 0.2) (layer "F.Cu") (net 41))
 (segment (start 94.0894 114.63) (end 92.8418 113.382) (width 0.2) (layer "F.Cu") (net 41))
 (via (at 92.8418 113.382) (size 0.6) (drill 0.3) (layers "F.Cu" "B.Cu") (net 41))
 (segment (start 93.4584 102.956) (end 94.0804 103.578) (width 0.2) (layer "B.Cu") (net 41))
 (segment (start 93.1 102) (end 93.1 102.956) (width 0.2) (layer "B.Cu") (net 41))
 (segment (start 93.4619 105) (end 92.7376 105) (width 0.2) (layer "B.Cu") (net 41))
 (segment (start 94.0804 103.578) (end 94.0804 104.382) (width 0.2) (layer "B.Cu") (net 41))
 (segment (start 92.1134 112.654) (end 92.8418 113.382) (width 0.2) (layer "B.Cu") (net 41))
 (segment (start 94.0804 104.382) (end 93.4619 105) (width 0.2) (layer "B.Cu") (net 41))
 (segment (start 93.1 102.956) (end 93.4584 102.956) (width 0.2) (layer "B.Cu") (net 41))
 (segment (start 92.7376 105) (end 92.1134 105.624) (width 0.2) (layer "B.Cu") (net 41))
 (segment (start 92.1134 105.624) (end 92.1134 112.654) (width 0.2) (layer "B.Cu") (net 41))
 (segment (start 100.98 98.12) (end 103.1 98.12) (width 0.2) (layer "F.Cu") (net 9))
 (segment (start 93.1 106) (end 100.98 98.12) (width 0.2) (layer "F.Cu") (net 9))
 (segment (start 138.062 112.002) (end 138.76 112.7) (width 0.2) (layer "F.Cu") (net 40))
 (segment (start 93.1024 112.002) (end 138.062 112.002) (width 0.2) (layer "F.Cu") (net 40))
 (segment (start 93.1 112) (end 93.1024 112.002) (width 0.2) (layer "F.Cu") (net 40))
 (segment (start 155.307 114.007) (end 155.307 118.328) (width 0.2) (layer "F.Cu") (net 29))
 (segment (start 154 112.7) (end 155.307 114.007) (width 0.2) (layer "F.Cu") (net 29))
 (segment (start 154.246 119.39) (end 130.322 119.39) (width 0.2) (layer "F.Cu") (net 29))
 (segment (start 155.307 118.328) (end 154.246 119.39) (width 0.2) (layer "F.Cu") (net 29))
 (via (at 130.322 119.39) (size 0.6) (drill 0.3) (layers "F.Cu" "B.Cu") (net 29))
 (segment (start 127.49 109.29) (end 127.49 113.845) (width 0.2) (layer "B.Cu") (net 29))
 (segment (start 130.322 116.293) (end 130.322 119.39) (width 0.2) (layer "B.Cu") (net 29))
 (segment (start 128.5 108.28) (end 127.49 109.29) (width 0.2) (layer "B.Cu") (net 29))
 (segment (start 128.275 114.63) (end 128.659 114.63) (width 0.2) (layer "B.Cu") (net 29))
 (segment (start 127.49 113.845) (end 128.275 114.63) (width 0.2) (layer "B.Cu") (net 29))
 (segment (start 128.659 114.63) (end 130.322 116.293) (width 0.2) (layer "B.Cu") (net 29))
 (segment (start 147.595 98.6752) (end 137.65 98.6752) (width 0.2) (layer "F.Cu") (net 31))
 (segment (start 137.65 98.6752) (end 133.99 102.336) (width 0.2) (layer "F.Cu") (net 31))
 (segment (start 154 105.08) (end 147.595 98.6752) (width 0.2) (layer "F.Cu") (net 31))
 (segment (start 133.99 102.336) (end 133.219 102.336) (width 0.2) (layer "F.Cu") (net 31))
 (via (at 133.219 102.336) (size 0.6) (drill 0.3) (layers "F.Cu" "B.Cu") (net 31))
 (segment (start 133.219 108.641) (end 128.5 113.36) (width 0.2) (layer "B.Cu") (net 31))
 (segment (start 133.219 102.336) (end 133.219 108.641) (width 0.2) (layer "B.Cu") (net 31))
 (segment (start 137.306 97.8839) (end 133.816 97.8839) (width 0.2) (layer "F.Cu") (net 27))
 (segment (start 137.461 97.7285) (end 137.306 97.8839) (width 0.2) (layer "F.Cu") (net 27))
 (segment (start 133.816 97.8839) (end 128.5 103.2) (width 0.2) (layer "F.Cu") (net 27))
 (segment (start 151.493 97.4931) (end 137.696 97.4931) (width 0.2) (layer "F.Cu") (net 27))
 (segment (start 137.696 97.4931) (end 137.461 97.7285) (width 0.2) (layer "F.Cu") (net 27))
 (segment (start 137.461 97.7285) (end 137.306 97.8839) (width 0.2) (layer "F.Cu") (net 27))
 (segment (start 154 100) (end 151.493 97.4931) (width 0.2) (layer "F.Cu") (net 27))
 (segment (start 142.888 85.42) (end 148.569 91.1012) (width 0.2) (layer "F.Cu") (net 20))
 (segment (start 128.5 85.42) (end 142.888 85.42) (width 0.2) (layer "F.Cu") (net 20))
 (via (at 148.569 91.1012) (size 0.6) (drill 0.3) (layers "F.Cu" "B.Cu") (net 20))
 (segment (start 148.569 102.189) (end 154 107.62) (width 0.2) (layer "B.Cu") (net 20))
 (segment (start 148.569 91.1012) (end 148.569 102.189) (width 0.2) (layer "B.Cu") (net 20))
 (segment (start 154 110.16) (end 142.467 110.16) (width 0.2) (layer "F.Cu") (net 30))
 (segment (start 141.832 110.795) (end 142.467 110.16) (width 0.2) (layer "F.Cu") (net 30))
 (segment (start 129.081 111.401) (end 128.5 110.82) (width 0.2) (layer "F.Cu") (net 30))
 (segment (start 137.356 111.401) (end 129.081 111.401) (width 0.2) (layer "F.Cu") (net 30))
 (segment (start 137.74 111.401) (end 137.356 111.401) (width 0.2) (layer "F.Cu") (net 30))
 (segment (start 142.467 110.16) (end 141.832 110.795) (width 0.2) (layer "F.Cu") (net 30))
 (segment (start 137.356 111.401) (end 137.74 111.401) (width 0.2) (layer "F.Cu") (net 30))
 (segment (start 137.74 111.401) (end 137.356 111.401) (width 0.2) (layer "F.Cu") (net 30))
 (segment (start 142.467 110.16) (end 141.832 110.795) (width 0.2) (layer "F.Cu") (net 30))
 (via (at 141.832 110.795) (size 0.6) (drill 0.3) (layers "F.Cu" "B.Cu") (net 30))
 (via (at 137.74 111.401) (size 0.6) (drill 0.3) (layers "F.Cu" "B.Cu") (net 30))
 (segment (start 137.468 111.672) (end 137.74 111.401) (width 0.2) (layer "B.Cu") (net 30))
 (segment (start 138.197 119.077) (end 137.468 118.348) (width 0.2) (layer "B.Cu") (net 30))
 (segment (start 141.832 110.795) (end 141.832 116.576) (width 0.2) (layer "B.Cu") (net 30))
 (segment (start 139.331 119.077) (end 138.197 119.077) (width 0.2) (layer "B.Cu") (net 30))
 (segment (start 137.468 118.348) (end 137.468 111.672) (width 0.2) (layer "B.Cu") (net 30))
 (segment (start 141.832 116.576) (end 139.331 119.077) (width 0.2) (layer "B.Cu") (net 30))
 (segment (start 137.53 97.0914) (end 153.298 97.0914) (width 0.2) (layer "F.Cu") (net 26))
 (segment (start 137.295 97.3268) (end 137.53 97.0914) (width 0.2) (layer "F.Cu") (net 26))
 (segment (start 131.735 97.4248) (end 128.5 100.66) (width 0.2) (layer "F.Cu") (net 26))
 (segment (start 137.295 97.3268) (end 137.197 97.4248) (width 0.2) (layer "F.Cu") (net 26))
 (segment (start 153.298 97.0914) (end 154.427 98.2208) (width 0.2) (layer "F.Cu") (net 26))
 (segment (start 137.197 97.4248) (end 131.735 97.4248) (width 0.2) (layer "F.Cu") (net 26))
 (segment (start 137.295 97.3268) (end 137.197 97.4248) (width 0.2) (layer "F.Cu") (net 26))
 (via (at 154.427 98.2208) (size 0.6) (drill 0.3) (layers "F.Cu" "B.Cu") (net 26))
 (segment (start 154.427 96.1081) (end 148.818 90.4995) (width 0.2) (layer "B.Cu") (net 26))
 (segment (start 148.818 90.4995) (end 148.32 90.4995) (width 0.2) (layer "B.Cu") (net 26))
 (segment (start 148.32 90.4995) (end 147.967 90.8521) (width 0.2) (layer "B.Cu") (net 26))
 (segment (start 154.427 98.2208) (end 154.427 96.1081) (width 0.2) (layer "B.Cu") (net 26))
 (segment (start 147.967 109.207) (end 154 115.24) (width 0.2) (layer "B.Cu") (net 26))
 (segment (start 147.967 90.8521) (end 147.967 109.207) (width 0.2) (layer "B.Cu") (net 26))
 (segment (start 137.863 97.8948) (end 137.061 98.6967) (width 0.2) (layer "F.Cu") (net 28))
 (segment (start 137.061 98.6967) (end 135.543 98.6967) (width 0.2) (layer "F.Cu") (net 28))
 (segment (start 149.355 97.8948) (end 137.863 97.8948) (width 0.2) (layer "F.Cu") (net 28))
 (segment (start 154 102.54) (end 149.355 97.8948) (width 0.2) (layer "F.Cu") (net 28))
 (segment (start 135.543 98.6967) (end 128.5 105.74) (width 0.2) (layer "F.Cu") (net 28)))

